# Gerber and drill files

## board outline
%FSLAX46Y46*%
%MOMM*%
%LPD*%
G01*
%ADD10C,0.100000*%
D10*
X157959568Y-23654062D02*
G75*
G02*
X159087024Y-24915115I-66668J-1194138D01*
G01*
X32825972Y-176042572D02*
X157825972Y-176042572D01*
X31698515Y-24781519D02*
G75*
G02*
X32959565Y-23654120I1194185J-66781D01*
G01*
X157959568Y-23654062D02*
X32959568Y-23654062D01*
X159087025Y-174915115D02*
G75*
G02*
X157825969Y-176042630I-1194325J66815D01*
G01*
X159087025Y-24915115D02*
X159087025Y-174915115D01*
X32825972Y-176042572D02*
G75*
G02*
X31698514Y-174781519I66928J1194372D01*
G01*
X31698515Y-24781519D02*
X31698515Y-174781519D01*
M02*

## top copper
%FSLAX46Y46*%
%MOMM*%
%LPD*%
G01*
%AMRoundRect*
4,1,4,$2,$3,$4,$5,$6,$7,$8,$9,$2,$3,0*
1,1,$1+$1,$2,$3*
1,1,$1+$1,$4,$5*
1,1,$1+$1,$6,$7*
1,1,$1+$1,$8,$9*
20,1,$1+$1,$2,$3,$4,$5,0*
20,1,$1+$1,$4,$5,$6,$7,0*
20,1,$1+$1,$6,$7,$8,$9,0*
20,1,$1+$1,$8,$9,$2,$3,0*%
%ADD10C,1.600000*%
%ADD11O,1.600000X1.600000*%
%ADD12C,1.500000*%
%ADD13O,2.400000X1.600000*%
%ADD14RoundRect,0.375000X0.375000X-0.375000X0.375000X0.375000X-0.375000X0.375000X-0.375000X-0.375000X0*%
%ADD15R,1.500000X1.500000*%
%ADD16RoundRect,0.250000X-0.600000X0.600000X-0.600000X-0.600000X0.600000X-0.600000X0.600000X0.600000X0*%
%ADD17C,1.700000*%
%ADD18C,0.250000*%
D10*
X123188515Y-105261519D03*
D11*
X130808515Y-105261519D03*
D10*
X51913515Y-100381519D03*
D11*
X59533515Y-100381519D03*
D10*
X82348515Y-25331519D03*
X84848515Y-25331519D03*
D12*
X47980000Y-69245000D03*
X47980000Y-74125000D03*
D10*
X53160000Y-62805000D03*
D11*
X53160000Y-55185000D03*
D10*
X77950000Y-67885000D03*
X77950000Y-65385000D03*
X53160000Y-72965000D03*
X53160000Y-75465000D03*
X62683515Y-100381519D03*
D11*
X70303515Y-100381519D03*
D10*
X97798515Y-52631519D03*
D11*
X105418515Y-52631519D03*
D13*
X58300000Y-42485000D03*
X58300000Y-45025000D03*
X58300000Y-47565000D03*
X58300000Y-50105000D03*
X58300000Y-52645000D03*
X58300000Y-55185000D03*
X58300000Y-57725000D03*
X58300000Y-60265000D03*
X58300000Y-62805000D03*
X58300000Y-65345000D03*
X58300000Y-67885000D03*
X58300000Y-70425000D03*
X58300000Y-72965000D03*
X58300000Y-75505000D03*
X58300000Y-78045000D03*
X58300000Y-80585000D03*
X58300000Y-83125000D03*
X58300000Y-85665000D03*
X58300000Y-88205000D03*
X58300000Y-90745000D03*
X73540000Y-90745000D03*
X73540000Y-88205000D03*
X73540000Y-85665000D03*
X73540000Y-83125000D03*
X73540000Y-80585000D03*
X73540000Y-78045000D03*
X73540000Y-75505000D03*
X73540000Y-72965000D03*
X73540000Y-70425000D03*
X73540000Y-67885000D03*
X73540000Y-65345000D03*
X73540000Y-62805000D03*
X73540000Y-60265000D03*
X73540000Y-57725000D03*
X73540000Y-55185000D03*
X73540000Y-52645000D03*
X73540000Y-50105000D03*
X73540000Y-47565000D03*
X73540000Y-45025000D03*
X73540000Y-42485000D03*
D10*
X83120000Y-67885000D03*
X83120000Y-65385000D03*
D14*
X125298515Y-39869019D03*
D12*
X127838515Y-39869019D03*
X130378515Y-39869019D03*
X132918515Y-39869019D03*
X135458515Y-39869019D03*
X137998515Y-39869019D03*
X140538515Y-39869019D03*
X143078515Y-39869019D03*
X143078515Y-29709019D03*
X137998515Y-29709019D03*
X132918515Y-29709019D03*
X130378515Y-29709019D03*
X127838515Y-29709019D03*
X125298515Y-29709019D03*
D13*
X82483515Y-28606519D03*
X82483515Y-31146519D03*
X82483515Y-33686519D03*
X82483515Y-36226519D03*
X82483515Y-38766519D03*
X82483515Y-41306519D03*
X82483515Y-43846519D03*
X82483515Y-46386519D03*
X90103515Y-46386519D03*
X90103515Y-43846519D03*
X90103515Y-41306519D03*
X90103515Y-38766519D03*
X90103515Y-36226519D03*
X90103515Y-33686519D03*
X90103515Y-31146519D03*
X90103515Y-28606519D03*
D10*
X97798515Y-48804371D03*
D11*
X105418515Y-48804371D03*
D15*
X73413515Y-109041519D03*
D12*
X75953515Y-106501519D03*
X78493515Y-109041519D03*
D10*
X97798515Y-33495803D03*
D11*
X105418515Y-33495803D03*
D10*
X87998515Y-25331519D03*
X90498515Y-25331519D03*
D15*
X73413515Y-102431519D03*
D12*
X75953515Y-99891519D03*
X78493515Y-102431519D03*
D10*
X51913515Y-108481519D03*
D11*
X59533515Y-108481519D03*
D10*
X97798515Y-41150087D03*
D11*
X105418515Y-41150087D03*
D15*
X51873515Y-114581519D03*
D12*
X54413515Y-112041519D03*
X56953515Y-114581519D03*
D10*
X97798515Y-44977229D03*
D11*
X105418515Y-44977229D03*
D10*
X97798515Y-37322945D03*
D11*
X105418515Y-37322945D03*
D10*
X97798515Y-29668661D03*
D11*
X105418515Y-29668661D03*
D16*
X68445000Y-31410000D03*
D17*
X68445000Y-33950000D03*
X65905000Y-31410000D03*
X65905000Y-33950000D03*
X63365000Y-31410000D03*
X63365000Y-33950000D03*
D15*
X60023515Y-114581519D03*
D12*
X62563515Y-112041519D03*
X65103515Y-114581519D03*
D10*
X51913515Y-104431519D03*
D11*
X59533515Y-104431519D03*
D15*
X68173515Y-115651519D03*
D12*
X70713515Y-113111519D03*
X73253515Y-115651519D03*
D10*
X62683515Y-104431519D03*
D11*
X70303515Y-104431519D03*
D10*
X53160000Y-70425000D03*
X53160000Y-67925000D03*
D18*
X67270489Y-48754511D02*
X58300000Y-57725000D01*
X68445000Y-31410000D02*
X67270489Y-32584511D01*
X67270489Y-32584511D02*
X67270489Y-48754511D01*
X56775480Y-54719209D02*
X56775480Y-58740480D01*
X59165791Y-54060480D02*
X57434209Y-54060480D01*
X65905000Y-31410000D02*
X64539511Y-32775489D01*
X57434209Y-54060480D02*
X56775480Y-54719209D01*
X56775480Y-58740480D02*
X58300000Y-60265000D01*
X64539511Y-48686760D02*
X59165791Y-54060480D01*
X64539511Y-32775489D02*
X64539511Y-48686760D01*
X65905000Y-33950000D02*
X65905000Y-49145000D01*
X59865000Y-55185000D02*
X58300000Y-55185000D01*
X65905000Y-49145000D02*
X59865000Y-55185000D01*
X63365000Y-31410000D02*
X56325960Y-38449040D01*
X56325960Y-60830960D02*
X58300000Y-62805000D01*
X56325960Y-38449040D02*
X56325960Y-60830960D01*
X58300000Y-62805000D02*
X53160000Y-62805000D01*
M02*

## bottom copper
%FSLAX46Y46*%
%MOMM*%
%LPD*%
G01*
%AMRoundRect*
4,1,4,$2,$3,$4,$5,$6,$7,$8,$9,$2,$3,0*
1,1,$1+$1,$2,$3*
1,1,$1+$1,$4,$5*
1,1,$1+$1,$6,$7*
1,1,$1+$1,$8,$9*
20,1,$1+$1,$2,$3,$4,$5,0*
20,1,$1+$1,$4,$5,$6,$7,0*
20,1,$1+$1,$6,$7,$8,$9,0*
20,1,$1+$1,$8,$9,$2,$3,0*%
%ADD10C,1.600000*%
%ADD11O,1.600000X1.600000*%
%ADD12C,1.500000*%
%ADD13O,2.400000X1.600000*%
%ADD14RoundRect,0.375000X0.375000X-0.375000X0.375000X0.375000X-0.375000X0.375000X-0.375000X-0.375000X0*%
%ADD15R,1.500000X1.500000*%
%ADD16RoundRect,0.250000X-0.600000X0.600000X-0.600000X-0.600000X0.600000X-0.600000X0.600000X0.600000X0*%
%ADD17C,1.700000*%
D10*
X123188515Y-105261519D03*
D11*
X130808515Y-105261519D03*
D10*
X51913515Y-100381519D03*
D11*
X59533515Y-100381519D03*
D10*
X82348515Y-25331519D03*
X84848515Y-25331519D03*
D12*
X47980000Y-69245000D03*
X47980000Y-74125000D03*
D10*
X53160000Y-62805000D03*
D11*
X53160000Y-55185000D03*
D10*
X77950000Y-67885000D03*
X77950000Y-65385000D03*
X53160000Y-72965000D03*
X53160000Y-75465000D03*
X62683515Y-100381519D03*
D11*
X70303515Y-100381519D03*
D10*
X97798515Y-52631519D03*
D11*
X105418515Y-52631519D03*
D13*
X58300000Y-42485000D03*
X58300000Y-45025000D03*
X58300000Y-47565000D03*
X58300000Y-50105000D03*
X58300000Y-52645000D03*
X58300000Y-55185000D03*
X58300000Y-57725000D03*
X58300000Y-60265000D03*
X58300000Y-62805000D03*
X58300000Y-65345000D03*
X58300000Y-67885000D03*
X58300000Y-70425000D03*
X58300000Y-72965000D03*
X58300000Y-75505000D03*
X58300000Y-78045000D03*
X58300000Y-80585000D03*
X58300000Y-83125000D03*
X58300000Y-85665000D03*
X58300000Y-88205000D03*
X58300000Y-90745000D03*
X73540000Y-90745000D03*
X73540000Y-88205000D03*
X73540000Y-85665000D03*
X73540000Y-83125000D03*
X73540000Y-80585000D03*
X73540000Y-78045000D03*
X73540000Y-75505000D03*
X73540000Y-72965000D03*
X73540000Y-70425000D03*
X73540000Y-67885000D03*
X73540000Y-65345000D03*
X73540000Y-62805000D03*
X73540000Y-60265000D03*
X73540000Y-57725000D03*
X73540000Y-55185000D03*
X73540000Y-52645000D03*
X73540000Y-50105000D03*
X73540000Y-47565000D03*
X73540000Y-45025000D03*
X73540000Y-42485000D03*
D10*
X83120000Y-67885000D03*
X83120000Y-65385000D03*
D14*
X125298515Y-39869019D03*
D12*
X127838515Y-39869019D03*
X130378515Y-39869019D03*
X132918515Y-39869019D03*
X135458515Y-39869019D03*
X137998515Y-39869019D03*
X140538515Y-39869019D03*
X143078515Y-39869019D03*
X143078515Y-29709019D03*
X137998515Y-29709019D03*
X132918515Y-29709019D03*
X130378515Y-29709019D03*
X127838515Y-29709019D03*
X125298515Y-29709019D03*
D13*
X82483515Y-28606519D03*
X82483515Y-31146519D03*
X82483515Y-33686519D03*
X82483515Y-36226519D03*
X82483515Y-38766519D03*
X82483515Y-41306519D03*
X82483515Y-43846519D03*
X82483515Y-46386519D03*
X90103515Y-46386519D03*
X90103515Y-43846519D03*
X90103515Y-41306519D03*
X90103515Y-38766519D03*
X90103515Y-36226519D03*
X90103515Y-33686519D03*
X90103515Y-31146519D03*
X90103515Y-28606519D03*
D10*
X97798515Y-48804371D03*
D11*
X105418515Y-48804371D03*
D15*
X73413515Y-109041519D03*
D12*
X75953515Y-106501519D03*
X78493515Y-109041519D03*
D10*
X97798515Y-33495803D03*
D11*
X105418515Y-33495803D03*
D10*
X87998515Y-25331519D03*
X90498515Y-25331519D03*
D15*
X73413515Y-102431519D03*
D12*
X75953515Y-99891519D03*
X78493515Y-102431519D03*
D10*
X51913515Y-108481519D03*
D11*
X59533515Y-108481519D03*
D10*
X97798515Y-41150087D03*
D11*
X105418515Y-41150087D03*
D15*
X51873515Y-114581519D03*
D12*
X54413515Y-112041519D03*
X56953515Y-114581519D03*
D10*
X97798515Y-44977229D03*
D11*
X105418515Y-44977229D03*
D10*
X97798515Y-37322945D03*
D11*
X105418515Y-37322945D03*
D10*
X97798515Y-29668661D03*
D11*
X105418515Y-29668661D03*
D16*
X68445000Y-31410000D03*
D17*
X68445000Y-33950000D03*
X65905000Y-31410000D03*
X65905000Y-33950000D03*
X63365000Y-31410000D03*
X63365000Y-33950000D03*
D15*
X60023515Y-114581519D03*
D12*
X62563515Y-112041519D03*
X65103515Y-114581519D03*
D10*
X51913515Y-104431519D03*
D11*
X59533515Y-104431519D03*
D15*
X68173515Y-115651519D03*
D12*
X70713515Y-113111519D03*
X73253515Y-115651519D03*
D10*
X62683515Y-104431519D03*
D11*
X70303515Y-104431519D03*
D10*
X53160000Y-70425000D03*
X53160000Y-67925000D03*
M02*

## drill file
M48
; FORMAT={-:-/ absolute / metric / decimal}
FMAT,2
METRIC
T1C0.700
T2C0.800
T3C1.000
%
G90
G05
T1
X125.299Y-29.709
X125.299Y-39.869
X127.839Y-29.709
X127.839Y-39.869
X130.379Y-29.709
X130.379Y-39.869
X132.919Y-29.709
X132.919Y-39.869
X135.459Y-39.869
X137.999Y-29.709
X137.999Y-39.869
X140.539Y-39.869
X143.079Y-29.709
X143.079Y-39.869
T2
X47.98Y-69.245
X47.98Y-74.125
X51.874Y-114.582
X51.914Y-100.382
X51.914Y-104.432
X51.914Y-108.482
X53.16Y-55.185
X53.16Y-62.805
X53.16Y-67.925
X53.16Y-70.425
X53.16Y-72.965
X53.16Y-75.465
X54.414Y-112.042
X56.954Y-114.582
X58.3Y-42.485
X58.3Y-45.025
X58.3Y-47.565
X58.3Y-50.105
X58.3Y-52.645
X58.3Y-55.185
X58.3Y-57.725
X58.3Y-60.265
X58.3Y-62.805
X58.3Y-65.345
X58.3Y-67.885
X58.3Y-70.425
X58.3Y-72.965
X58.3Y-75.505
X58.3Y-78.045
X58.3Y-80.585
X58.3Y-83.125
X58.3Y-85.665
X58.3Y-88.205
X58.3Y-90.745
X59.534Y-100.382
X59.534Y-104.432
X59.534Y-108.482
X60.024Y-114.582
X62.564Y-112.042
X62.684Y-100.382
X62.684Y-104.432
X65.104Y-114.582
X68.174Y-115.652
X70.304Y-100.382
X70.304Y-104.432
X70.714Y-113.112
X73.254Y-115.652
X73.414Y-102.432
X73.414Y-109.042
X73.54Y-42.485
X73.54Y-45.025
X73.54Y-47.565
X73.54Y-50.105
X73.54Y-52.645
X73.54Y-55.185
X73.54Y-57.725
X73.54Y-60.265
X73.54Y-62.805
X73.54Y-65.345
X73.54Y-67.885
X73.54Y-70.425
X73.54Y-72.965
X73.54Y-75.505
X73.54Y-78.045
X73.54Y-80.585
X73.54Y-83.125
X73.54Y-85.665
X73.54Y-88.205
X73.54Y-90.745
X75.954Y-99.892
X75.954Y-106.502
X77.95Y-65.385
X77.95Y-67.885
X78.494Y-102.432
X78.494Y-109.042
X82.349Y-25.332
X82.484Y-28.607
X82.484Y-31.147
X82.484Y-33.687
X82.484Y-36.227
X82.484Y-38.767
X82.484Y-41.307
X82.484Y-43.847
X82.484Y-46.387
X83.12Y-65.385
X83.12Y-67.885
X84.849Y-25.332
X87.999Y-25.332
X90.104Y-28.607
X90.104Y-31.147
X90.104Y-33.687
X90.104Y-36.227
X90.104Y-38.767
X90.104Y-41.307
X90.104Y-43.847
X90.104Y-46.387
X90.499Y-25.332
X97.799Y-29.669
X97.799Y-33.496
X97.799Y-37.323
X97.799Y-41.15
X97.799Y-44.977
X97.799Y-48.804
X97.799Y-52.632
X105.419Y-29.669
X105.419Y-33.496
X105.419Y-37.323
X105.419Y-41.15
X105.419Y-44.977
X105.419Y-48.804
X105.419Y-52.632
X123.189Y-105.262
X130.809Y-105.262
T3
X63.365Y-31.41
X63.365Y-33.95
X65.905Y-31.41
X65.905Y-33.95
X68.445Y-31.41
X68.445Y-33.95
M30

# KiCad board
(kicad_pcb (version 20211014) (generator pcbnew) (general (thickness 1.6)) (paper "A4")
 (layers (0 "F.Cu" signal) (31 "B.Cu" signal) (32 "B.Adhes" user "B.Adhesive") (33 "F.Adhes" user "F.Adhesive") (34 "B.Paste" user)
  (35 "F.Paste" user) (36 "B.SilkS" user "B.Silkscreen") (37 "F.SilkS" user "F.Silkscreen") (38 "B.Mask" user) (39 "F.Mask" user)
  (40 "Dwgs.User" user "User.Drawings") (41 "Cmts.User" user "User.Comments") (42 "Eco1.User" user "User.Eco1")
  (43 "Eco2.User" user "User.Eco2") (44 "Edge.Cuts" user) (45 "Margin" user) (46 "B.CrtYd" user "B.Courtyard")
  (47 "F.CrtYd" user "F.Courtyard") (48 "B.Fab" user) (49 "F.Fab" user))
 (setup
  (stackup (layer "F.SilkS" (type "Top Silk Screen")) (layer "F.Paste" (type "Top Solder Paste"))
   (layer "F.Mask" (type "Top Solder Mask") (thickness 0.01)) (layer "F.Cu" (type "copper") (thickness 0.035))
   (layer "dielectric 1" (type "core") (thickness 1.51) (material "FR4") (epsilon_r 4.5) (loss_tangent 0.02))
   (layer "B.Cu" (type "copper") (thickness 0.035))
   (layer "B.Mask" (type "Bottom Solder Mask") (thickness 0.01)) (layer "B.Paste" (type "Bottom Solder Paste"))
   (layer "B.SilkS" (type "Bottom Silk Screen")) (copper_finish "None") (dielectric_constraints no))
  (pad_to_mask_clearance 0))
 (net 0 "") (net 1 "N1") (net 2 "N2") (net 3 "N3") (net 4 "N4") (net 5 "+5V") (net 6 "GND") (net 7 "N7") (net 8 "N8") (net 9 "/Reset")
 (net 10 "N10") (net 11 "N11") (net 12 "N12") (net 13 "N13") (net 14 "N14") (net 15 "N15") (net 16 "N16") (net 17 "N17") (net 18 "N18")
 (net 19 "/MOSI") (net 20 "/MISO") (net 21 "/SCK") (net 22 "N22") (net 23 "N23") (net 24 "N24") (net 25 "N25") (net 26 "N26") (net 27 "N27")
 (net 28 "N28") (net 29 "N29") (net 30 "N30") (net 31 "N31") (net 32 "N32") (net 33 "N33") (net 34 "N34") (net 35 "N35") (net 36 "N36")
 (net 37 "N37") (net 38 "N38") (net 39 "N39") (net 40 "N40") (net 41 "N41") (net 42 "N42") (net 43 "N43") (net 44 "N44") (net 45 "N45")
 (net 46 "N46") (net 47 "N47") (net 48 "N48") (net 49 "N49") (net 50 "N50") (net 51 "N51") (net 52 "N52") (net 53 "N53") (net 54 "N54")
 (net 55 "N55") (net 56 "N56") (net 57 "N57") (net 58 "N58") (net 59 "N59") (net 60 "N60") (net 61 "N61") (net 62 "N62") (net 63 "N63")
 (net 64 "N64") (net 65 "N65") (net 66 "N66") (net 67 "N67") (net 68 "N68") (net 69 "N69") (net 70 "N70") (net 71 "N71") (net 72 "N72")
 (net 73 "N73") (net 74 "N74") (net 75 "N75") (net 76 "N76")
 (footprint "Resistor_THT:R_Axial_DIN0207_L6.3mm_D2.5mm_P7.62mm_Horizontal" (layer "F.Cu") (at 123.188515 105.261519)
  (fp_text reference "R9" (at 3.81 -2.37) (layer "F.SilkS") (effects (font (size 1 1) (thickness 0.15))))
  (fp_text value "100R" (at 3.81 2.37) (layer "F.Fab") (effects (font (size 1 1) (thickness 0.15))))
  (pad "1" thru_hole circle (at 0 0) (size 1.6 1.6) (drill 0.8) (layers *.Cu *.Mask) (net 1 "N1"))
  (pad "2" thru_hole oval (at 7.62 0) (size 1.6 1.6) (drill 0.8) (layers *.Cu *.Mask) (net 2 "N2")))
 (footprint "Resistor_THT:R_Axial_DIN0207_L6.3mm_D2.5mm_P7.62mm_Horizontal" (layer "F.Cu") (at 51.913515 100.381519)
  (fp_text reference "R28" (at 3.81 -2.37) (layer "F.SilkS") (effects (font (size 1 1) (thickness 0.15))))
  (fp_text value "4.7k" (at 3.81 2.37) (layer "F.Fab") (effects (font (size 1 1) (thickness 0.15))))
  (pad "1" thru_hole circle (at 0 0) (size 1.6 1.6) (drill 0.8) (layers *.Cu *.Mask) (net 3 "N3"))
  (pad "2" thru_hole oval (at 7.62 0) (size 1.6 1.6) (drill 0.8) (layers *.Cu *.Mask) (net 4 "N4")))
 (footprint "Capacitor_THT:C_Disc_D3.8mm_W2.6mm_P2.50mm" (layer "F.Cu") (at 82.348515 25.331519)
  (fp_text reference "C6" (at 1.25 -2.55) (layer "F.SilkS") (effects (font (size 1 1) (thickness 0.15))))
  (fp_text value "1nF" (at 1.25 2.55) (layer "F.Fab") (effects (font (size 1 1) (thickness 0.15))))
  (pad "1" thru_hole circle (at 0 0) (size 1.6 1.6) (drill 0.8) (layers *.Cu *.Mask) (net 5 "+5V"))
  (pad "2" thru_hole circle (at 2.5 0) (size 1.6 1.6) (drill 0.8) (layers *.Cu *.Mask) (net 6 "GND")))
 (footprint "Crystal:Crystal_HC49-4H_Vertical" (layer "F.Cu") (at 47.98 69.245 -90)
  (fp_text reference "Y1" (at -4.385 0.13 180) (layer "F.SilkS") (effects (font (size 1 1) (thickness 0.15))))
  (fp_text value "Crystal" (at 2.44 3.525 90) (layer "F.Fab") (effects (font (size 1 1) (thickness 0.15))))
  (pad "1" thru_hole circle (at 0 0 270) (size 1.5 1.5) (drill 0.8) (layers *.Cu *.Mask) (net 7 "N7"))
  (pad "2" thru_hole circle (at 4.88 0 270) (size 1.5 1.5) (drill 0.8) (layers *.Cu *.Mask) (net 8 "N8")))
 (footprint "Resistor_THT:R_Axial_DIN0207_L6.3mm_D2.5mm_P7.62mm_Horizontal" (layer "F.Cu") (at 53.16 62.805 90)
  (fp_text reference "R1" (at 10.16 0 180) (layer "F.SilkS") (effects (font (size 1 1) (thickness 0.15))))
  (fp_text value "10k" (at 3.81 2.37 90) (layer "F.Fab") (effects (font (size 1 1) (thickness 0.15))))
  (pad "1" thru_hole circle (at 0 0 90) (size 1.6 1.6) (drill 0.8) (layers *.Cu *.Mask) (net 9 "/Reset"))
  (pad "2" thru_hole oval (at 7.62 0 90) (size 1.6 1.6) (drill 0.8) (layers *.Cu *.Mask) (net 5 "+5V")))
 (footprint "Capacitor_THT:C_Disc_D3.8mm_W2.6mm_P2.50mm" (layer "F.Cu") (at 77.95 67.885 90)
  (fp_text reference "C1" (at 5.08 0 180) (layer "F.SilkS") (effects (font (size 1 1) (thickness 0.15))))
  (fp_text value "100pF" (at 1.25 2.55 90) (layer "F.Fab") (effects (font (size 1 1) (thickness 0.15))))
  (pad "1" thru_hole circle (at 0 0 90) (size 1.6 1.6) (drill 0.8) (layers *.Cu *.Mask) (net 5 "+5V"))
  (pad "2" thru_hole circle (at 2.5 0 90) (size 1.6 1.6) (drill 0.8) (layers *.Cu *.Mask) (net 6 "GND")))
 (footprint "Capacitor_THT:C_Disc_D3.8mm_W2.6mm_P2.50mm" (layer "F.Cu") (at 53.16 72.965 -90)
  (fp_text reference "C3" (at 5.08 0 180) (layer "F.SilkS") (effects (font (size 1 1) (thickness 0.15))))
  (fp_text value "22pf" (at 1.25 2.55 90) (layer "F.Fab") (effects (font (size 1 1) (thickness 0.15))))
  (pad "1" thru_hole circle (at 0 0 270) (size 1.6 1.6) (drill 0.8) (layers *.Cu *.Mask) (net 8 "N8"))
  (pad "2" thru_hole circle (at 2.5 0 270) (size 1.6 1.6) (drill 0.8) (layers *.Cu *.Mask) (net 6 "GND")))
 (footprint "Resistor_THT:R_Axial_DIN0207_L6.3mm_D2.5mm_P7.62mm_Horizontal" (layer "F.Cu") (at 62.683515 100.381519)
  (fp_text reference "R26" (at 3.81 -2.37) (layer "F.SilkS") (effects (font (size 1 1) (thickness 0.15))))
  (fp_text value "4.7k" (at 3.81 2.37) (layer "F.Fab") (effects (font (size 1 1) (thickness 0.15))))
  (pad "1" thru_hole circle (at 0 0) (size 1.6 1.6) (drill 0.8) (layers *.Cu *.Mask) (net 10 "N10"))
  (pad "2" thru_hole oval (at 7.62 0) (size 1.6 1.6) (drill 0.8) (layers *.Cu *.Mask) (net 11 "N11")))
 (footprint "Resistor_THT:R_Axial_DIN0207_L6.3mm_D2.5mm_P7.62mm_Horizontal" (layer "F.Cu") (at 97.798515 52.631519)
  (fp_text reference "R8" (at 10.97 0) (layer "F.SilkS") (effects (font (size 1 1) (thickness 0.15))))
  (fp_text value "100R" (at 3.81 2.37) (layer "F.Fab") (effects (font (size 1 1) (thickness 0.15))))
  (pad "1" thru_hole circle (at 0 0) (size 1.6 1.6) (drill 0.8) (layers *.Cu *.Mask) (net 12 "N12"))
  (pad "2" thru_hole oval (at 7.62 0) (size 1.6 1.6) (drill 0.8) (layers *.Cu *.Mask) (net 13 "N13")))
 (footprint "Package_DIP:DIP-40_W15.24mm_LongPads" (layer "F.Cu") (at 58.3 42.485)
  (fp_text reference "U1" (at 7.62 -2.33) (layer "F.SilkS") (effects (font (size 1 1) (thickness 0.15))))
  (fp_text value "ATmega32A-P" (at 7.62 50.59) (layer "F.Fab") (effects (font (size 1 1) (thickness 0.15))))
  (pad "1" thru_hole oval (at 0 0) (size 2.4 1.6) (drill 0.8) (layers *.Cu *.Mask) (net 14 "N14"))
  (pad "2" thru_hole oval (at 0 2.54) (size 2.4 1.6) (drill 0.8) (layers *.Cu *.Mask) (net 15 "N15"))
  (pad "3" thru_hole oval (at 0 5.08) (size 2.4 1.6) (drill 0.8) (layers *.Cu *.Mask) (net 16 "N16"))
  (pad "4" thru_hole oval (at 0 7.62) (size 2.4 1.6) (drill 0.8) (layers *.Cu *.Mask) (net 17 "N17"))
  (pad "5" thru_hole oval (at 0 10.16) (size 2.4 1.6) (drill 0.8) (layers *.Cu *.Mask) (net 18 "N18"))
  (pad "6" thru_hole oval (at 0 12.7) (size 2.4 1.6) (drill 0.8) (layers *.Cu *.Mask) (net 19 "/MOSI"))
  (pad "7" thru_hole oval (at 0 15.24) (size 2.4 1.6) (drill 0.8) (layers *.Cu *.Mask) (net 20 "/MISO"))
  (pad "8" thru_hole oval (at 0 17.78) (size 2.4 1.6) (drill 0.8) (layers *.Cu *.Mask) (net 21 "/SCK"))
  (pad "9" thru_hole oval (at 0 20.32) (size 2.4 1.6) (drill 0.8) (layers *.Cu *.Mask) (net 9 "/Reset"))
  (pad "10" thru_hole oval (at 0 22.86) (size 2.4 1.6) (drill 0.8) (layers *.Cu *.Mask) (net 5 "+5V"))
  (pad "11" thru_hole oval (at 0 25.4) (size 2.4 1.6) (drill 0.8) (layers *.Cu *.Mask) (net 6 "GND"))
  (pad "12" thru_hole oval (at 0 27.94) (size 2.4 1.6) (drill 0.8) (layers *.Cu *.Mask) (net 7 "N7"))
  (pad "13" thru_hole oval (at 0 30.48) (size 2.4 1.6) (drill 0.8) (layers *.Cu *.Mask) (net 8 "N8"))
  (pad "14" thru_hole oval (at 0 33.02) (size 2.4 1.6) (drill 0.8) (layers *.Cu *.Mask) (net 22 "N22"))
  (pad "15" thru_hole oval (at 0 35.56) (size 2.4 1.6) (drill 0.8) (layers *.Cu *.Mask) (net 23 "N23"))
  (pad "16" thru_hole oval (at 0 38.1) (size 2.4 1.6) (drill 0.8) (layers *.Cu *.Mask) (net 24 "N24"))
  (pad "17" thru_hole oval (at 0 40.64) (size 2.4 1.6) (drill 0.8) (layers *.Cu *.Mask) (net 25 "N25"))
  (pad "18" thru_hole oval (at 0 43.18) (size 2.4 1.6) (drill 0.8) (layers *.Cu *.Mask) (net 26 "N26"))
  (pad "19" thru_hole oval (at 0 45.72) (size 2.4 1.6) (drill 0.8) (layers *.Cu *.Mask) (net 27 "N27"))
  (pad "20" thru_hole oval (at 0 48.26) (size 2.4 1.6) (drill 0.8) (layers *.Cu *.Mask) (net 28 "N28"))
  (pad "21" thru_hole oval (at 15.24 48.26) (size 2.4 1.6) (drill 0.8) (layers *.Cu *.Mask) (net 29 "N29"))
  (pad "22" thru_hole oval (at 15.24 45.72) (size 2.4 1.6) (drill 0.8) (layers *.Cu *.Mask) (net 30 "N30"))
  (pad "23" thru_hole oval (at 15.24 43.18) (size 2.4 1.6) (drill 0.8) (layers *.Cu *.Mask) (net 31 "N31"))
  (pad "24" thru_hole oval (at 15.24 40.64) (size 2.4 1.6) (drill 0.8) (layers *.Cu *.Mask) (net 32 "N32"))
  (pad "25" thru_hole oval (at 15.24 38.1) (size 2.4 1.6) (drill 0.8) (layers *.Cu *.Mask) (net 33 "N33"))
  (pad "26" thru_hole oval (at 15.24 35.56) (size 2.4 1.6) (drill 0.8) (layers *.Cu *.Mask) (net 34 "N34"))
  (pad "27" thru_hole oval (at 15.24 33.02) (size 2.4 1.6) (drill 0.8) (layers *.Cu *.Mask) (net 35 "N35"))
  (pad "28" thru_hole oval (at 15.24 30.48) (size 2.4 1.6) (drill 0.8) (layers *.Cu *.Mask) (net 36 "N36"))
  (pad "29" thru_hole oval (at 15.24 27.94) (size 2.4 1.6) (drill 0.8) (layers *.Cu *.Mask) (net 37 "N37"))
  (pad "30" thru_hole oval (at 15.24 25.4) (size 2.4 1.6) (drill 0.8) (layers *.Cu *.Mask) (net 5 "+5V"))
  (pad "31" thru_hole oval (at 15.24 22.86) (size 2.4 1.6) (drill 0.8) (layers *.Cu *.Mask) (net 6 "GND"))
  (pad "32" thru_hole oval (at 15.24 20.32) (size 2.4 1.6) (drill 0.8) (layers *.Cu *.Mask) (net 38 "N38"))
  (pad "33" thru_hole oval (at 15.24 17.78) (size 2.4 1.6) (drill 0.8) (layers *.Cu *.Mask) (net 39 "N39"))
  (pad "34" thru_hole oval (at 15.24 15.24) (size 2.4 1.6) (drill 0.8) (layers *.Cu *.Mask) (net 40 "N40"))
  (pad "35" thru_hole oval (at 15.24 12.7) (size 2.4 1.6) (drill 0.8) (layers *.Cu *.Mask) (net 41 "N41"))
  (pad "36" thru_hole oval (at 15.24 10.16) (size 2.4 1.6) (drill 0.8) (layers *.Cu *.Mask) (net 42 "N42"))
  (pad "37" thru_hole oval (at 15.24 7.62) (size 2.4 1.6) (drill 0.8) (layers *.Cu *.Mask) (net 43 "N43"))
  (pad "38" thru_hole oval (at 15.24 5.08) (size 2.4 1.6) (drill 0.8) (layers *.Cu *.Mask) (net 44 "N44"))
  (pad "39" thru_hole oval (at 15.24 2.54) (size 2.4 1.6) (drill 0.8) (layers *.Cu *.Mask) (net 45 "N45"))
  (pad "40" thru_hole oval (at 15.24 0) (size 2.4 1.6) (drill 0.8) (layers *.Cu *.Mask) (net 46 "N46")))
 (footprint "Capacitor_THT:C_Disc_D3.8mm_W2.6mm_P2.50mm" (layer "F.Cu") (at 83.12 67.885 90)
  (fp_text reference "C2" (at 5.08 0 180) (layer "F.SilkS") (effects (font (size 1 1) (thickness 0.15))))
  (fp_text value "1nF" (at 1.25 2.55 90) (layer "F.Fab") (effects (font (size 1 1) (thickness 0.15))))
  (pad "1" thru_hole circle (at 0 0 90) (size 1.6 1.6) (drill 0.8) (layers *.Cu *.Mask) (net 5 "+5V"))
  (pad "2" thru_hole circle (at 2.5 0 90) (size 1.6 1.6) (drill 0.8) (layers *.Cu *.Mask) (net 6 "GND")))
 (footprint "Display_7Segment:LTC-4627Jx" (layer "F.Cu") (at 125.298515 39.869019 90)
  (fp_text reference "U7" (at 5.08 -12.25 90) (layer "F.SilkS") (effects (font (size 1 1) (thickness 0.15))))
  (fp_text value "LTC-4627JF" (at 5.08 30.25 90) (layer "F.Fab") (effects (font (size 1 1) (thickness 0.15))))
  (pad "1" thru_hole roundrect (at 0 0 90) (size 1.5 1.5) (drill 0.7) (layers *.Cu *.Mask) (roundrect_rratio 0.25) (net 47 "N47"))
  (pad "2" thru_hole circle (at 0 2.54 90) (size 1.5 1.5) (drill 0.7) (layers *.Cu *.Mask) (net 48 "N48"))
  (pad "3" thru_hole circle (at 0 5.08 90) (size 1.5 1.5) (drill 0.7) (layers *.Cu *.Mask) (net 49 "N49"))
  (pad "4" thru_hole circle (at 0 7.62 90) (size 1.5 1.5) (drill 0.7) (layers *.Cu *.Mask) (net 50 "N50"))
  (pad "5" thru_hole circle (at 0 10.16 90) (size 1.5 1.5) (drill 0.7) (layers *.Cu *.Mask) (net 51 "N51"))
  (pad "6" thru_hole circle (at 0 12.7 90) (size 1.5 1.5) (drill 0.7) (layers *.Cu *.Mask) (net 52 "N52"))
  (pad "7" thru_hole circle (at 0 15.24 90) (size 1.5 1.5) (drill 0.7) (layers *.Cu *.Mask) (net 2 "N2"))
  (pad "8" thru_hole circle (at 0 17.78 90) (size 1.5 1.5) (drill 0.7) (layers *.Cu *.Mask) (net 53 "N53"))
  (pad "9" thru_hole circle (at 10.16 17.78 90) (size 1.5 1.5) (drill 0.7) (layers *.Cu *.Mask) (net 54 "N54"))
  (pad "11" thru_hole circle (at 10.16 12.7 90) (size 1.5 1.5) (drill 0.7) (layers *.Cu *.Mask) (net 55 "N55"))
  (pad "13" thru_hole circle (at 10.16 7.62 90) (size 1.5 1.5) (drill 0.7) (layers *.Cu *.Mask) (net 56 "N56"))
  (pad "14" thru_hole circle (at 10.16 5.08 90) (size 1.5 1.5) (drill 0.7) (layers *.Cu *.Mask) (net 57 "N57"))
  (pad "15" thru_hole circle (at 10.16 2.54 90) (size 1.5 1.5) (drill 0.7) (layers *.Cu *.Mask) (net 13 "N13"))
  (pad "16" thru_hole circle (at 10.16 0 90) (size 1.5 1.5) (drill 0.7) (layers *.Cu *.Mask) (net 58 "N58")))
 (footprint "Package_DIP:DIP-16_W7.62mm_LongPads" (layer "F.Cu") (at 82.483515 28.606519)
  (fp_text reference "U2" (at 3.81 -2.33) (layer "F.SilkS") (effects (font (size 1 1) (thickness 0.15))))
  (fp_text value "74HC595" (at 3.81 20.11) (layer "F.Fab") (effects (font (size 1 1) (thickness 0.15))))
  (pad "1" thru_hole oval (at 0 0) (size 2.4 1.6) (drill 0.8) (layers *.Cu *.Mask) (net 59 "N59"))
  (pad "2" thru_hole oval (at 0 2.54) (size 2.4 1.6) (drill 0.8) (layers *.Cu *.Mask) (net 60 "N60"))
  (pad "3" thru_hole oval (at 0 5.08) (size 2.4 1.6) (drill 0.8) (layers *.Cu *.Mask) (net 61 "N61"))
  (pad "4" thru_hole oval (at 0 7.62) (size 2.4 1.6) (drill 0.8) (layers *.Cu *.Mask) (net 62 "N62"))
  (pad "5" thru_hole oval (at 0 10.16) (size 2.4 1.6) (drill 0.8) (layers *.Cu *.Mask) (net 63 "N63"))
  (pad "6" thru_hole oval (at 0 12.7) (size 2.4 1.6) (drill 0.8) (layers *.Cu *.Mask) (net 12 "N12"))
  (pad "7" thru_hole oval (at 0 15.24) (size 2.4 1.6) (drill 0.8) (layers *.Cu *.Mask) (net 1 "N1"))
  (pad "8" thru_hole oval (at 0 17.78) (size 2.4 1.6) (drill 0.8) (layers *.Cu *.Mask) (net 6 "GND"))
  (pad "9" thru_hole oval (at 7.62 17.78) (size 2.4 1.6) (drill 0.8) (layers *.Cu *.Mask) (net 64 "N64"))
  (pad "10" thru_hole oval (at 7.62 15.24) (size 2.4 1.6) (drill 0.8) (layers *.Cu *.Mask) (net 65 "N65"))
  (pad "11" thru_hole oval (at 7.62 12.7) (size 2.4 1.6) (drill 0.8) (layers *.Cu *.Mask) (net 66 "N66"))
  (pad "12" thru_hole oval (at 7.62 10.16) (size 2.4 1.6) (drill 0.8) (layers *.Cu *.Mask) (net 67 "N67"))
  (pad "13" thru_hole oval (at 7.62 7.62) (size 2.4 1.6) (drill 0.8) (layers *.Cu *.Mask) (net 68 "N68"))
  (pad "14" thru_hole oval (at 7.62 5.08) (size 2.4 1.6) (drill 0.8) (layers *.Cu *.Mask) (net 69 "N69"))
  (pad "15" thru_hole oval (at 7.62 2.54) (size 2.4 1.6) (drill 0.8) (layers *.Cu *.Mask) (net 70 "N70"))
  (pad "16" thru_hole oval (at 7.62 0) (size 2.4 1.6) (drill 0.8) (layers *.Cu *.Mask) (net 5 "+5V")))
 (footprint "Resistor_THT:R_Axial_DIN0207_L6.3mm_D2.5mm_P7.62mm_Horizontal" (layer "F.Cu") (at 97.798515 48.804371)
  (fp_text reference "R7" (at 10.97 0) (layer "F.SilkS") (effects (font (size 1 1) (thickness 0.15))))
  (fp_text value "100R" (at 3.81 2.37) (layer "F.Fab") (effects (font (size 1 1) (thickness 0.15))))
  (pad "1" thru_hole circle (at 0 0) (size 1.6 1.6) (drill 0.8) (layers *.Cu *.Mask) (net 63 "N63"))
  (pad "2" thru_hole oval (at 7.62 0) (size 1.6 1.6) (drill 0.8) (layers *.Cu *.Mask) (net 55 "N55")))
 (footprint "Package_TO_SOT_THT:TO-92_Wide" (layer "F.Cu") (at 73.413515 109.041519)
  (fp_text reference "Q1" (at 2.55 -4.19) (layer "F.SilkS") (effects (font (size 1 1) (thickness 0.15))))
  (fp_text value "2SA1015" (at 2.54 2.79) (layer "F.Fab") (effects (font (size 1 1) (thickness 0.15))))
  (pad "1" thru_hole rect (at 0 0) (size 1.5 1.5) (drill 0.8) (layers *.Cu *.Mask) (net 5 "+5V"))
  (pad "2" thru_hole circle (at 2.54 -2.54) (size 1.5 1.5) (drill 0.8) (layers *.Cu *.Mask) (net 47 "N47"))
  (pad "3" thru_hole circle (at 5.08 0) (size 1.5 1.5) (drill 0.8) (layers *.Cu *.Mask) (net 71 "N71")))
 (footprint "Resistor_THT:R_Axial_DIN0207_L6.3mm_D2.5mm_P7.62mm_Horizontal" (layer "F.Cu") (at 97.798515 33.495803)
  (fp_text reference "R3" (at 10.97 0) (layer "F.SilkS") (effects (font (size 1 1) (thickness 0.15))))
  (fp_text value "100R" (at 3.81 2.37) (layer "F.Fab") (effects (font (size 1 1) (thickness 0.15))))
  (pad "1" thru_hole circle (at 0 0) (size 1.6 1.6) (drill 0.8) (layers *.Cu *.Mask) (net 59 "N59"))
  (pad "2" thru_hole oval (at 7.62 0) (size 1.6 1.6) (drill 0.8) (layers *.Cu *.Mask) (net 58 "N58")))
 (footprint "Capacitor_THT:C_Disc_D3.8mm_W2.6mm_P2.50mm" (layer "F.Cu") (at 87.998515 25.331519)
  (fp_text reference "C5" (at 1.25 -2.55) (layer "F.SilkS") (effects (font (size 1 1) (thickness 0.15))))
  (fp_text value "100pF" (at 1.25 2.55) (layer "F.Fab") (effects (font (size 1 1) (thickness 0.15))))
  (pad "1" thru_hole circle (at 0 0) (size 1.6 1.6) (drill 0.8) (layers *.Cu *.Mask) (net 5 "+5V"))
  (pad "2" thru_hole circle (at 2.5 0) (size 1.6 1.6) (drill 0.8) (layers *.Cu *.Mask) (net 6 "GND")))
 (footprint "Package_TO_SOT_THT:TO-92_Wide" (layer "F.Cu") (at 73.413515 102.431519)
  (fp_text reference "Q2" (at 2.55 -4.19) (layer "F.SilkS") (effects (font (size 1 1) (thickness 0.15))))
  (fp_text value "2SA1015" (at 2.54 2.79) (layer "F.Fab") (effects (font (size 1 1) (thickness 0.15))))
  (pad "1" thru_hole rect (at 0 0) (size 1.5 1.5) (drill 0.8) (layers *.Cu *.Mask) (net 5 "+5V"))
  (pad "2" thru_hole circle (at 2.54 -2.54) (size 1.5 1.5) (drill 0.8) (layers *.Cu *.Mask) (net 48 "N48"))
  (pad "3" thru_hole circle (at 5.08 0) (size 1.5 1.5) (drill 0.8) (layers *.Cu *.Mask) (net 11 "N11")))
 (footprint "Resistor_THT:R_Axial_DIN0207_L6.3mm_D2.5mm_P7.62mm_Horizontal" (layer "F.Cu") (at 51.913515 108.481519)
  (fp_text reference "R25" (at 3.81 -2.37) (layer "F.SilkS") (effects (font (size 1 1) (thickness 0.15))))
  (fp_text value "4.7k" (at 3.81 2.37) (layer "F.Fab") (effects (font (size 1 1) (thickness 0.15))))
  (pad "1" thru_hole circle (at 0 0) (size 1.6 1.6) (drill 0.8) (layers *.Cu *.Mask) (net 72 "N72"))
  (pad "2" thru_hole oval (at 7.62 0) (size 1.6 1.6) (drill 0.8) (layers *.Cu *.Mask) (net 71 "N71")))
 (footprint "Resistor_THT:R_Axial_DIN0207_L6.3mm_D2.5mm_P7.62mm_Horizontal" (layer "F.Cu") (at 97.798515 41.150087)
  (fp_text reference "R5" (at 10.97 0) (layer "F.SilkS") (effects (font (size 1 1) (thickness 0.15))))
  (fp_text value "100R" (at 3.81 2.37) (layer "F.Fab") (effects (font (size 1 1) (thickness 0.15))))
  (pad "1" thru_hole circle (at 0 0) (size 1.6 1.6) (drill 0.8) (layers *.Cu *.Mask) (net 61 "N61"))
  (pad "2" thru_hole oval (at 7.62 0) (size 1.6 1.6) (drill 0.8) (layers *.Cu *.Mask) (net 49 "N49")))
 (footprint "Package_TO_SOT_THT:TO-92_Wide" (layer "F.Cu") (at 51.873515 114.581519)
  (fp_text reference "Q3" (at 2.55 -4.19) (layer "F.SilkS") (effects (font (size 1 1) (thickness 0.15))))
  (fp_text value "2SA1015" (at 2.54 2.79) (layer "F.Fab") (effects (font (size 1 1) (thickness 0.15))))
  (pad "1" thru_hole rect (at 0 0) (size 1.5 1.5) (drill 0.8) (layers *.Cu *.Mask) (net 5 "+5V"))
  (pad "2" thru_hole circle (at 2.54 -2.54) (size 1.5 1.5) (drill 0.8) (layers *.Cu *.Mask) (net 52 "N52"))
  (pad "3" thru_hole circle (at 5.08 0) (size 1.5 1.5) (drill 0.8) (layers *.Cu *.Mask) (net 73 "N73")))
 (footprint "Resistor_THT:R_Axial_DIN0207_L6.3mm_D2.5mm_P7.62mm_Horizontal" (layer "F.Cu") (at 97.798515 44.977229)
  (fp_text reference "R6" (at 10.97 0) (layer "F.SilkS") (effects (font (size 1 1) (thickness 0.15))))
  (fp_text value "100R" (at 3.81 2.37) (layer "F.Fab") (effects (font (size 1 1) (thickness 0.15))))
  (pad "1" thru_hole circle (at 0 0) (size 1.6 1.6) (drill 0.8) (layers *.Cu *.Mask) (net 62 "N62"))
  (pad "2" thru_hole oval (at 7.62 0) (size 1.6 1.6) (drill 0.8) (layers *.Cu *.Mask) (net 51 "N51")))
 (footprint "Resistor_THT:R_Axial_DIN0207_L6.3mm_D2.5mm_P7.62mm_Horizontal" (layer "F.Cu") (at 97.798515 37.322945)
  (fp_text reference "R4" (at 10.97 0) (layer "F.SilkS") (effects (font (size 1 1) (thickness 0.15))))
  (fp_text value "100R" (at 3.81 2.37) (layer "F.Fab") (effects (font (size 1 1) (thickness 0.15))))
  (pad "1" thru_hole circle (at 0 0) (size 1.6 1.6) (drill 0.8) (layers *.Cu *.Mask) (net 60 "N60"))
  (pad "2" thru_hole oval (at 7.62 0) (size 1.6 1.6) (drill 0.8) (layers *.Cu *.Mask) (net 56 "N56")))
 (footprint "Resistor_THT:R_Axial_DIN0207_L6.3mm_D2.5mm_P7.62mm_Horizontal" (layer "F.Cu") (at 97.798515 29.668661)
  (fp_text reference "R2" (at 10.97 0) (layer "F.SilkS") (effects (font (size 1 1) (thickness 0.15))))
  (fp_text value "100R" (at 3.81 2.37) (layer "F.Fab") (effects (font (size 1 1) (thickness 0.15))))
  (pad "1" thru_hole circle (at 0 0) (size 1.6 1.6) (drill 0.8) (layers *.Cu *.Mask) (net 70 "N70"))
  (pad "2" thru_hole oval (at 7.62 0) (size 1.6 1.6) (drill 0.8) (layers *.Cu *.Mask) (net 57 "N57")))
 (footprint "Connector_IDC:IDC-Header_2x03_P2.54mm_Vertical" (layer "F.Cu") (at 68.445 31.41 -90)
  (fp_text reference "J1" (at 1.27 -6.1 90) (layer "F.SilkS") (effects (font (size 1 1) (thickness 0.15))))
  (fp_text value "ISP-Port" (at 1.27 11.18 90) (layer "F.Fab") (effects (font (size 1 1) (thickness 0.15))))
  (pad "1" thru_hole roundrect (at 0 0 270) (size 1.7 1.7) (drill 1) (layers *.Cu *.Mask) (roundrect_rratio 0.147059) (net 20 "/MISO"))
  (pad "2" thru_hole circle (at 2.54 0 270) (size 1.7 1.7) (drill 1) (layers *.Cu *.Mask) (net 5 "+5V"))
  (pad "3" thru_hole circle (at 0 2.54 270) (size 1.7 1.7) (drill 1) (layers *.Cu *.Mask) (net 21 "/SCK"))
  (pad "4" thru_hole circle (at 2.54 2.54 270) (size 1.7 1.7) (drill 1) (layers *.Cu *.Mask) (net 19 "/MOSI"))
  (pad "5" thru_hole circle (at 0 5.08 270) (size 1.7 1.7) (drill 1) (layers *.Cu *.Mask) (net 9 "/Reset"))
  (pad "6" thru_hole circle (at 2.54 5.08 270) (size 1.7 1.7) (drill 1) (layers *.Cu *.Mask) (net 6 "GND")))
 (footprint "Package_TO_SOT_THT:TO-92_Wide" (layer "F.Cu") (at 60.023515 114.581519)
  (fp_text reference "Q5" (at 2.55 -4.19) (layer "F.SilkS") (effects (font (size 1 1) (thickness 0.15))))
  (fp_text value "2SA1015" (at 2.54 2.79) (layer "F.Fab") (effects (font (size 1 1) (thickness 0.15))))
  (pad "1" thru_hole rect (at 0 0) (size 1.5 1.5) (drill 0.8) (layers *.Cu *.Mask) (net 5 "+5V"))
  (pad "2" thru_hole circle (at 2.54 -2.54) (size 1.5 1.5) (drill 0.8) (layers *.Cu *.Mask) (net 50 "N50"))
  (pad "3" thru_hole circle (at 5.08 0) (size 1.5 1.5) (drill 0.8) (layers *.Cu *.Mask) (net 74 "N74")))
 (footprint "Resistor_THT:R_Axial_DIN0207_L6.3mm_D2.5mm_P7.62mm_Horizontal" (layer "F.Cu") (at 51.913515 104.431519)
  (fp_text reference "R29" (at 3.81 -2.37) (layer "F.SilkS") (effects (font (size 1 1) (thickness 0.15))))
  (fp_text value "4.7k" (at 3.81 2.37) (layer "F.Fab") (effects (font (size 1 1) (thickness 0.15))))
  (pad "1" thru_hole circle (at 0 0) (size 1.6 1.6) (drill 0.8) (layers *.Cu *.Mask) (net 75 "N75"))
  (pad "2" thru_hole oval (at 7.62 0) (size 1.6 1.6) (drill 0.8) (layers *.Cu *.Mask) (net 74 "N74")))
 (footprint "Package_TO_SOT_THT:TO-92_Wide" (layer "F.Cu") (at 68.173515 115.651519)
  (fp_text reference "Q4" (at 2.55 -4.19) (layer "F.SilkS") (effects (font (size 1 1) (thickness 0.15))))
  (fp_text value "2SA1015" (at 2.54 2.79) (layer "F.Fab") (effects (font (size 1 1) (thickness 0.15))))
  (pad "1" thru_hole rect (at 0 0) (size 1.5 1.5) (drill 0.8) (layers *.Cu *.Mask) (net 5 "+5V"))
  (pad "2" thru_hole circle (at 2.54 -2.54) (size 1.5 1.5) (drill 0.8) (layers *.Cu *.Mask) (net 53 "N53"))
  (pad "3" thru_hole circle (at 5.08 0) (size 1.5 1.5) (drill 0.8) (layers *.Cu *.Mask) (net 4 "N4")))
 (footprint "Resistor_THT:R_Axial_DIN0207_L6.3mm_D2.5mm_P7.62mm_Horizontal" (layer "F.Cu") (at 62.683515 104.431519)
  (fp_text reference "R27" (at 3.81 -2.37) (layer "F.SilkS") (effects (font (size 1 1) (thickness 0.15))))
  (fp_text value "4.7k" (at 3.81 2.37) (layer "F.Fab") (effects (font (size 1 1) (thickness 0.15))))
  (pad "1" thru_hole circle (at 0 0) (size 1.6 1.6) (drill 0.8) (layers *.Cu *.Mask) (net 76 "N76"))
  (pad "2" thru_hole oval (at 7.62 0) (size 1.6 1.6) (drill 0.8) (layers *.Cu *.Mask) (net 73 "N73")))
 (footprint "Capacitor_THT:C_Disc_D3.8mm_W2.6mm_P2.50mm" (layer "F.Cu") (at 53.16 70.425 90)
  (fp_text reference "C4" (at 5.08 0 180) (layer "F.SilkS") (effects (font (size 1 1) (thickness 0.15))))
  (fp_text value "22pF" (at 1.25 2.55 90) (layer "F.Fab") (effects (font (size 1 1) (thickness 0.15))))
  (pad "1" thru_hole circle (at 0 0 90) (size 1.6 1.6) (drill 0.8) (layers *.Cu *.Mask) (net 7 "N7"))
  (pad "2" thru_hole circle (at 2.5 0 90) (size 1.6 1.6) (drill 0.8) (layers *.Cu *.Mask) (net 6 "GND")))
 (gr_arc locked (start 157.959568 23.654062) (mid 158.784499 24.05107) (end 159.087025 24.915115) (layer "Edge.Cuts") (width 0.1))
 (gr_line locked (start 32.825972 176.042572) (end 157.825972 176.042572) (layer "Edge.Cuts") (width 0.1))
 (gr_arc locked (start 31.698515 24.781519) (mid 32.095536 23.956601) (end 32.959568 23.654062) (layer "Edge.Cuts") (width 0.1))
 (gr_line locked (start 157.959568 23.654062) (end 32.959568 23.654062) (layer "Edge.Cuts") (width 0.1))
 (gr_arc locked (start 159.087025 174.915115) (mid 158.69 175.74) (end 157.825972 176.042572) (layer "Edge.Cuts") (width 0.1))
 (gr_line locked (start 159.087025 24.915115) (end 159.087025 174.915115) (layer "Edge.Cuts") (width 0.1))
 (gr_arc locked (start 32.825972 176.042572) (mid 32.001101 175.645535) (end 31.698515 174.781519) (layer "Edge.Cuts") (width 0.1))
 (gr_line locked (start 31.698515 24.781519) (end 31.698515 174.781519) (layer "Edge.Cuts") (width 0.1))
 (segment (start 67.270489 48.754511) (end 58.3 57.725) (width 0.25) (layer "F.Cu") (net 20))
 (segment (start 68.445 31.41) (end 67.270489 32.584511) (width 0.25) (layer "F.Cu") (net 20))
 (segment (start 67.270489 32.584511) (end 67.270489 48.754511) (width 0.25) (layer "F.Cu") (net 20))
 (segment (start 56.77548 54.719209) (end 56.77548 58.74048) (width 0.25) (layer "F.Cu") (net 21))
 (segment (start 59.165791 54.06048) (end 57.434209 54.06048) (width 0.25) (layer "F.Cu") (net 21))
 (segment (start 65.905 31.41) (end 64.539511 32.775489) (width 0.25) (layer "F.Cu") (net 21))
 (segment (start 57.434209 54.06048) (end 56.77548 54.719209) (width 0.25) (layer "F.Cu") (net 21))
 (segment (start 56.77548 58.74048) (end 58.3 60.265) (width 0.25) (layer "F.Cu") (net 21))
 (segment (start 64.539511 48.68676) (end 59.165791 54.06048) (width 0.25) (layer "F.Cu") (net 21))
 (segment (start 64.539511 32.775489) (end 64.539511 48.68676) (width 0.25) (layer "F.Cu") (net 21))
 (segment (start 65.905 33.95) (end 65.905 49.145) (width 0.25) (layer "F.Cu") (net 19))
 (segment (start 59.865 55.185) (end 58.3 55.185) (width 0.25) (layer "F.Cu") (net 19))
 (segment (start 65.905 49.145) (end 59.865 55.185) (width 0.25) (layer "F.Cu") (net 19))
 (segment (start 63.365 31.41) (end 56.32596 38.44904) (width 0.25) (layer "F.Cu") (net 9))
 (segment (start 56.32596 60.83096) (end 58.3 62.805) (width 0.25) (layer "F.Cu") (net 9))
 (segment (start 56.32596 38.44904) (end 56.32596 60.83096) (width 0.25) (layer "F.Cu") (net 9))
 (segment (start 58.3 62.805) (end 53.16 62.805) (width 0.25) (layer "F.Cu") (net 9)))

